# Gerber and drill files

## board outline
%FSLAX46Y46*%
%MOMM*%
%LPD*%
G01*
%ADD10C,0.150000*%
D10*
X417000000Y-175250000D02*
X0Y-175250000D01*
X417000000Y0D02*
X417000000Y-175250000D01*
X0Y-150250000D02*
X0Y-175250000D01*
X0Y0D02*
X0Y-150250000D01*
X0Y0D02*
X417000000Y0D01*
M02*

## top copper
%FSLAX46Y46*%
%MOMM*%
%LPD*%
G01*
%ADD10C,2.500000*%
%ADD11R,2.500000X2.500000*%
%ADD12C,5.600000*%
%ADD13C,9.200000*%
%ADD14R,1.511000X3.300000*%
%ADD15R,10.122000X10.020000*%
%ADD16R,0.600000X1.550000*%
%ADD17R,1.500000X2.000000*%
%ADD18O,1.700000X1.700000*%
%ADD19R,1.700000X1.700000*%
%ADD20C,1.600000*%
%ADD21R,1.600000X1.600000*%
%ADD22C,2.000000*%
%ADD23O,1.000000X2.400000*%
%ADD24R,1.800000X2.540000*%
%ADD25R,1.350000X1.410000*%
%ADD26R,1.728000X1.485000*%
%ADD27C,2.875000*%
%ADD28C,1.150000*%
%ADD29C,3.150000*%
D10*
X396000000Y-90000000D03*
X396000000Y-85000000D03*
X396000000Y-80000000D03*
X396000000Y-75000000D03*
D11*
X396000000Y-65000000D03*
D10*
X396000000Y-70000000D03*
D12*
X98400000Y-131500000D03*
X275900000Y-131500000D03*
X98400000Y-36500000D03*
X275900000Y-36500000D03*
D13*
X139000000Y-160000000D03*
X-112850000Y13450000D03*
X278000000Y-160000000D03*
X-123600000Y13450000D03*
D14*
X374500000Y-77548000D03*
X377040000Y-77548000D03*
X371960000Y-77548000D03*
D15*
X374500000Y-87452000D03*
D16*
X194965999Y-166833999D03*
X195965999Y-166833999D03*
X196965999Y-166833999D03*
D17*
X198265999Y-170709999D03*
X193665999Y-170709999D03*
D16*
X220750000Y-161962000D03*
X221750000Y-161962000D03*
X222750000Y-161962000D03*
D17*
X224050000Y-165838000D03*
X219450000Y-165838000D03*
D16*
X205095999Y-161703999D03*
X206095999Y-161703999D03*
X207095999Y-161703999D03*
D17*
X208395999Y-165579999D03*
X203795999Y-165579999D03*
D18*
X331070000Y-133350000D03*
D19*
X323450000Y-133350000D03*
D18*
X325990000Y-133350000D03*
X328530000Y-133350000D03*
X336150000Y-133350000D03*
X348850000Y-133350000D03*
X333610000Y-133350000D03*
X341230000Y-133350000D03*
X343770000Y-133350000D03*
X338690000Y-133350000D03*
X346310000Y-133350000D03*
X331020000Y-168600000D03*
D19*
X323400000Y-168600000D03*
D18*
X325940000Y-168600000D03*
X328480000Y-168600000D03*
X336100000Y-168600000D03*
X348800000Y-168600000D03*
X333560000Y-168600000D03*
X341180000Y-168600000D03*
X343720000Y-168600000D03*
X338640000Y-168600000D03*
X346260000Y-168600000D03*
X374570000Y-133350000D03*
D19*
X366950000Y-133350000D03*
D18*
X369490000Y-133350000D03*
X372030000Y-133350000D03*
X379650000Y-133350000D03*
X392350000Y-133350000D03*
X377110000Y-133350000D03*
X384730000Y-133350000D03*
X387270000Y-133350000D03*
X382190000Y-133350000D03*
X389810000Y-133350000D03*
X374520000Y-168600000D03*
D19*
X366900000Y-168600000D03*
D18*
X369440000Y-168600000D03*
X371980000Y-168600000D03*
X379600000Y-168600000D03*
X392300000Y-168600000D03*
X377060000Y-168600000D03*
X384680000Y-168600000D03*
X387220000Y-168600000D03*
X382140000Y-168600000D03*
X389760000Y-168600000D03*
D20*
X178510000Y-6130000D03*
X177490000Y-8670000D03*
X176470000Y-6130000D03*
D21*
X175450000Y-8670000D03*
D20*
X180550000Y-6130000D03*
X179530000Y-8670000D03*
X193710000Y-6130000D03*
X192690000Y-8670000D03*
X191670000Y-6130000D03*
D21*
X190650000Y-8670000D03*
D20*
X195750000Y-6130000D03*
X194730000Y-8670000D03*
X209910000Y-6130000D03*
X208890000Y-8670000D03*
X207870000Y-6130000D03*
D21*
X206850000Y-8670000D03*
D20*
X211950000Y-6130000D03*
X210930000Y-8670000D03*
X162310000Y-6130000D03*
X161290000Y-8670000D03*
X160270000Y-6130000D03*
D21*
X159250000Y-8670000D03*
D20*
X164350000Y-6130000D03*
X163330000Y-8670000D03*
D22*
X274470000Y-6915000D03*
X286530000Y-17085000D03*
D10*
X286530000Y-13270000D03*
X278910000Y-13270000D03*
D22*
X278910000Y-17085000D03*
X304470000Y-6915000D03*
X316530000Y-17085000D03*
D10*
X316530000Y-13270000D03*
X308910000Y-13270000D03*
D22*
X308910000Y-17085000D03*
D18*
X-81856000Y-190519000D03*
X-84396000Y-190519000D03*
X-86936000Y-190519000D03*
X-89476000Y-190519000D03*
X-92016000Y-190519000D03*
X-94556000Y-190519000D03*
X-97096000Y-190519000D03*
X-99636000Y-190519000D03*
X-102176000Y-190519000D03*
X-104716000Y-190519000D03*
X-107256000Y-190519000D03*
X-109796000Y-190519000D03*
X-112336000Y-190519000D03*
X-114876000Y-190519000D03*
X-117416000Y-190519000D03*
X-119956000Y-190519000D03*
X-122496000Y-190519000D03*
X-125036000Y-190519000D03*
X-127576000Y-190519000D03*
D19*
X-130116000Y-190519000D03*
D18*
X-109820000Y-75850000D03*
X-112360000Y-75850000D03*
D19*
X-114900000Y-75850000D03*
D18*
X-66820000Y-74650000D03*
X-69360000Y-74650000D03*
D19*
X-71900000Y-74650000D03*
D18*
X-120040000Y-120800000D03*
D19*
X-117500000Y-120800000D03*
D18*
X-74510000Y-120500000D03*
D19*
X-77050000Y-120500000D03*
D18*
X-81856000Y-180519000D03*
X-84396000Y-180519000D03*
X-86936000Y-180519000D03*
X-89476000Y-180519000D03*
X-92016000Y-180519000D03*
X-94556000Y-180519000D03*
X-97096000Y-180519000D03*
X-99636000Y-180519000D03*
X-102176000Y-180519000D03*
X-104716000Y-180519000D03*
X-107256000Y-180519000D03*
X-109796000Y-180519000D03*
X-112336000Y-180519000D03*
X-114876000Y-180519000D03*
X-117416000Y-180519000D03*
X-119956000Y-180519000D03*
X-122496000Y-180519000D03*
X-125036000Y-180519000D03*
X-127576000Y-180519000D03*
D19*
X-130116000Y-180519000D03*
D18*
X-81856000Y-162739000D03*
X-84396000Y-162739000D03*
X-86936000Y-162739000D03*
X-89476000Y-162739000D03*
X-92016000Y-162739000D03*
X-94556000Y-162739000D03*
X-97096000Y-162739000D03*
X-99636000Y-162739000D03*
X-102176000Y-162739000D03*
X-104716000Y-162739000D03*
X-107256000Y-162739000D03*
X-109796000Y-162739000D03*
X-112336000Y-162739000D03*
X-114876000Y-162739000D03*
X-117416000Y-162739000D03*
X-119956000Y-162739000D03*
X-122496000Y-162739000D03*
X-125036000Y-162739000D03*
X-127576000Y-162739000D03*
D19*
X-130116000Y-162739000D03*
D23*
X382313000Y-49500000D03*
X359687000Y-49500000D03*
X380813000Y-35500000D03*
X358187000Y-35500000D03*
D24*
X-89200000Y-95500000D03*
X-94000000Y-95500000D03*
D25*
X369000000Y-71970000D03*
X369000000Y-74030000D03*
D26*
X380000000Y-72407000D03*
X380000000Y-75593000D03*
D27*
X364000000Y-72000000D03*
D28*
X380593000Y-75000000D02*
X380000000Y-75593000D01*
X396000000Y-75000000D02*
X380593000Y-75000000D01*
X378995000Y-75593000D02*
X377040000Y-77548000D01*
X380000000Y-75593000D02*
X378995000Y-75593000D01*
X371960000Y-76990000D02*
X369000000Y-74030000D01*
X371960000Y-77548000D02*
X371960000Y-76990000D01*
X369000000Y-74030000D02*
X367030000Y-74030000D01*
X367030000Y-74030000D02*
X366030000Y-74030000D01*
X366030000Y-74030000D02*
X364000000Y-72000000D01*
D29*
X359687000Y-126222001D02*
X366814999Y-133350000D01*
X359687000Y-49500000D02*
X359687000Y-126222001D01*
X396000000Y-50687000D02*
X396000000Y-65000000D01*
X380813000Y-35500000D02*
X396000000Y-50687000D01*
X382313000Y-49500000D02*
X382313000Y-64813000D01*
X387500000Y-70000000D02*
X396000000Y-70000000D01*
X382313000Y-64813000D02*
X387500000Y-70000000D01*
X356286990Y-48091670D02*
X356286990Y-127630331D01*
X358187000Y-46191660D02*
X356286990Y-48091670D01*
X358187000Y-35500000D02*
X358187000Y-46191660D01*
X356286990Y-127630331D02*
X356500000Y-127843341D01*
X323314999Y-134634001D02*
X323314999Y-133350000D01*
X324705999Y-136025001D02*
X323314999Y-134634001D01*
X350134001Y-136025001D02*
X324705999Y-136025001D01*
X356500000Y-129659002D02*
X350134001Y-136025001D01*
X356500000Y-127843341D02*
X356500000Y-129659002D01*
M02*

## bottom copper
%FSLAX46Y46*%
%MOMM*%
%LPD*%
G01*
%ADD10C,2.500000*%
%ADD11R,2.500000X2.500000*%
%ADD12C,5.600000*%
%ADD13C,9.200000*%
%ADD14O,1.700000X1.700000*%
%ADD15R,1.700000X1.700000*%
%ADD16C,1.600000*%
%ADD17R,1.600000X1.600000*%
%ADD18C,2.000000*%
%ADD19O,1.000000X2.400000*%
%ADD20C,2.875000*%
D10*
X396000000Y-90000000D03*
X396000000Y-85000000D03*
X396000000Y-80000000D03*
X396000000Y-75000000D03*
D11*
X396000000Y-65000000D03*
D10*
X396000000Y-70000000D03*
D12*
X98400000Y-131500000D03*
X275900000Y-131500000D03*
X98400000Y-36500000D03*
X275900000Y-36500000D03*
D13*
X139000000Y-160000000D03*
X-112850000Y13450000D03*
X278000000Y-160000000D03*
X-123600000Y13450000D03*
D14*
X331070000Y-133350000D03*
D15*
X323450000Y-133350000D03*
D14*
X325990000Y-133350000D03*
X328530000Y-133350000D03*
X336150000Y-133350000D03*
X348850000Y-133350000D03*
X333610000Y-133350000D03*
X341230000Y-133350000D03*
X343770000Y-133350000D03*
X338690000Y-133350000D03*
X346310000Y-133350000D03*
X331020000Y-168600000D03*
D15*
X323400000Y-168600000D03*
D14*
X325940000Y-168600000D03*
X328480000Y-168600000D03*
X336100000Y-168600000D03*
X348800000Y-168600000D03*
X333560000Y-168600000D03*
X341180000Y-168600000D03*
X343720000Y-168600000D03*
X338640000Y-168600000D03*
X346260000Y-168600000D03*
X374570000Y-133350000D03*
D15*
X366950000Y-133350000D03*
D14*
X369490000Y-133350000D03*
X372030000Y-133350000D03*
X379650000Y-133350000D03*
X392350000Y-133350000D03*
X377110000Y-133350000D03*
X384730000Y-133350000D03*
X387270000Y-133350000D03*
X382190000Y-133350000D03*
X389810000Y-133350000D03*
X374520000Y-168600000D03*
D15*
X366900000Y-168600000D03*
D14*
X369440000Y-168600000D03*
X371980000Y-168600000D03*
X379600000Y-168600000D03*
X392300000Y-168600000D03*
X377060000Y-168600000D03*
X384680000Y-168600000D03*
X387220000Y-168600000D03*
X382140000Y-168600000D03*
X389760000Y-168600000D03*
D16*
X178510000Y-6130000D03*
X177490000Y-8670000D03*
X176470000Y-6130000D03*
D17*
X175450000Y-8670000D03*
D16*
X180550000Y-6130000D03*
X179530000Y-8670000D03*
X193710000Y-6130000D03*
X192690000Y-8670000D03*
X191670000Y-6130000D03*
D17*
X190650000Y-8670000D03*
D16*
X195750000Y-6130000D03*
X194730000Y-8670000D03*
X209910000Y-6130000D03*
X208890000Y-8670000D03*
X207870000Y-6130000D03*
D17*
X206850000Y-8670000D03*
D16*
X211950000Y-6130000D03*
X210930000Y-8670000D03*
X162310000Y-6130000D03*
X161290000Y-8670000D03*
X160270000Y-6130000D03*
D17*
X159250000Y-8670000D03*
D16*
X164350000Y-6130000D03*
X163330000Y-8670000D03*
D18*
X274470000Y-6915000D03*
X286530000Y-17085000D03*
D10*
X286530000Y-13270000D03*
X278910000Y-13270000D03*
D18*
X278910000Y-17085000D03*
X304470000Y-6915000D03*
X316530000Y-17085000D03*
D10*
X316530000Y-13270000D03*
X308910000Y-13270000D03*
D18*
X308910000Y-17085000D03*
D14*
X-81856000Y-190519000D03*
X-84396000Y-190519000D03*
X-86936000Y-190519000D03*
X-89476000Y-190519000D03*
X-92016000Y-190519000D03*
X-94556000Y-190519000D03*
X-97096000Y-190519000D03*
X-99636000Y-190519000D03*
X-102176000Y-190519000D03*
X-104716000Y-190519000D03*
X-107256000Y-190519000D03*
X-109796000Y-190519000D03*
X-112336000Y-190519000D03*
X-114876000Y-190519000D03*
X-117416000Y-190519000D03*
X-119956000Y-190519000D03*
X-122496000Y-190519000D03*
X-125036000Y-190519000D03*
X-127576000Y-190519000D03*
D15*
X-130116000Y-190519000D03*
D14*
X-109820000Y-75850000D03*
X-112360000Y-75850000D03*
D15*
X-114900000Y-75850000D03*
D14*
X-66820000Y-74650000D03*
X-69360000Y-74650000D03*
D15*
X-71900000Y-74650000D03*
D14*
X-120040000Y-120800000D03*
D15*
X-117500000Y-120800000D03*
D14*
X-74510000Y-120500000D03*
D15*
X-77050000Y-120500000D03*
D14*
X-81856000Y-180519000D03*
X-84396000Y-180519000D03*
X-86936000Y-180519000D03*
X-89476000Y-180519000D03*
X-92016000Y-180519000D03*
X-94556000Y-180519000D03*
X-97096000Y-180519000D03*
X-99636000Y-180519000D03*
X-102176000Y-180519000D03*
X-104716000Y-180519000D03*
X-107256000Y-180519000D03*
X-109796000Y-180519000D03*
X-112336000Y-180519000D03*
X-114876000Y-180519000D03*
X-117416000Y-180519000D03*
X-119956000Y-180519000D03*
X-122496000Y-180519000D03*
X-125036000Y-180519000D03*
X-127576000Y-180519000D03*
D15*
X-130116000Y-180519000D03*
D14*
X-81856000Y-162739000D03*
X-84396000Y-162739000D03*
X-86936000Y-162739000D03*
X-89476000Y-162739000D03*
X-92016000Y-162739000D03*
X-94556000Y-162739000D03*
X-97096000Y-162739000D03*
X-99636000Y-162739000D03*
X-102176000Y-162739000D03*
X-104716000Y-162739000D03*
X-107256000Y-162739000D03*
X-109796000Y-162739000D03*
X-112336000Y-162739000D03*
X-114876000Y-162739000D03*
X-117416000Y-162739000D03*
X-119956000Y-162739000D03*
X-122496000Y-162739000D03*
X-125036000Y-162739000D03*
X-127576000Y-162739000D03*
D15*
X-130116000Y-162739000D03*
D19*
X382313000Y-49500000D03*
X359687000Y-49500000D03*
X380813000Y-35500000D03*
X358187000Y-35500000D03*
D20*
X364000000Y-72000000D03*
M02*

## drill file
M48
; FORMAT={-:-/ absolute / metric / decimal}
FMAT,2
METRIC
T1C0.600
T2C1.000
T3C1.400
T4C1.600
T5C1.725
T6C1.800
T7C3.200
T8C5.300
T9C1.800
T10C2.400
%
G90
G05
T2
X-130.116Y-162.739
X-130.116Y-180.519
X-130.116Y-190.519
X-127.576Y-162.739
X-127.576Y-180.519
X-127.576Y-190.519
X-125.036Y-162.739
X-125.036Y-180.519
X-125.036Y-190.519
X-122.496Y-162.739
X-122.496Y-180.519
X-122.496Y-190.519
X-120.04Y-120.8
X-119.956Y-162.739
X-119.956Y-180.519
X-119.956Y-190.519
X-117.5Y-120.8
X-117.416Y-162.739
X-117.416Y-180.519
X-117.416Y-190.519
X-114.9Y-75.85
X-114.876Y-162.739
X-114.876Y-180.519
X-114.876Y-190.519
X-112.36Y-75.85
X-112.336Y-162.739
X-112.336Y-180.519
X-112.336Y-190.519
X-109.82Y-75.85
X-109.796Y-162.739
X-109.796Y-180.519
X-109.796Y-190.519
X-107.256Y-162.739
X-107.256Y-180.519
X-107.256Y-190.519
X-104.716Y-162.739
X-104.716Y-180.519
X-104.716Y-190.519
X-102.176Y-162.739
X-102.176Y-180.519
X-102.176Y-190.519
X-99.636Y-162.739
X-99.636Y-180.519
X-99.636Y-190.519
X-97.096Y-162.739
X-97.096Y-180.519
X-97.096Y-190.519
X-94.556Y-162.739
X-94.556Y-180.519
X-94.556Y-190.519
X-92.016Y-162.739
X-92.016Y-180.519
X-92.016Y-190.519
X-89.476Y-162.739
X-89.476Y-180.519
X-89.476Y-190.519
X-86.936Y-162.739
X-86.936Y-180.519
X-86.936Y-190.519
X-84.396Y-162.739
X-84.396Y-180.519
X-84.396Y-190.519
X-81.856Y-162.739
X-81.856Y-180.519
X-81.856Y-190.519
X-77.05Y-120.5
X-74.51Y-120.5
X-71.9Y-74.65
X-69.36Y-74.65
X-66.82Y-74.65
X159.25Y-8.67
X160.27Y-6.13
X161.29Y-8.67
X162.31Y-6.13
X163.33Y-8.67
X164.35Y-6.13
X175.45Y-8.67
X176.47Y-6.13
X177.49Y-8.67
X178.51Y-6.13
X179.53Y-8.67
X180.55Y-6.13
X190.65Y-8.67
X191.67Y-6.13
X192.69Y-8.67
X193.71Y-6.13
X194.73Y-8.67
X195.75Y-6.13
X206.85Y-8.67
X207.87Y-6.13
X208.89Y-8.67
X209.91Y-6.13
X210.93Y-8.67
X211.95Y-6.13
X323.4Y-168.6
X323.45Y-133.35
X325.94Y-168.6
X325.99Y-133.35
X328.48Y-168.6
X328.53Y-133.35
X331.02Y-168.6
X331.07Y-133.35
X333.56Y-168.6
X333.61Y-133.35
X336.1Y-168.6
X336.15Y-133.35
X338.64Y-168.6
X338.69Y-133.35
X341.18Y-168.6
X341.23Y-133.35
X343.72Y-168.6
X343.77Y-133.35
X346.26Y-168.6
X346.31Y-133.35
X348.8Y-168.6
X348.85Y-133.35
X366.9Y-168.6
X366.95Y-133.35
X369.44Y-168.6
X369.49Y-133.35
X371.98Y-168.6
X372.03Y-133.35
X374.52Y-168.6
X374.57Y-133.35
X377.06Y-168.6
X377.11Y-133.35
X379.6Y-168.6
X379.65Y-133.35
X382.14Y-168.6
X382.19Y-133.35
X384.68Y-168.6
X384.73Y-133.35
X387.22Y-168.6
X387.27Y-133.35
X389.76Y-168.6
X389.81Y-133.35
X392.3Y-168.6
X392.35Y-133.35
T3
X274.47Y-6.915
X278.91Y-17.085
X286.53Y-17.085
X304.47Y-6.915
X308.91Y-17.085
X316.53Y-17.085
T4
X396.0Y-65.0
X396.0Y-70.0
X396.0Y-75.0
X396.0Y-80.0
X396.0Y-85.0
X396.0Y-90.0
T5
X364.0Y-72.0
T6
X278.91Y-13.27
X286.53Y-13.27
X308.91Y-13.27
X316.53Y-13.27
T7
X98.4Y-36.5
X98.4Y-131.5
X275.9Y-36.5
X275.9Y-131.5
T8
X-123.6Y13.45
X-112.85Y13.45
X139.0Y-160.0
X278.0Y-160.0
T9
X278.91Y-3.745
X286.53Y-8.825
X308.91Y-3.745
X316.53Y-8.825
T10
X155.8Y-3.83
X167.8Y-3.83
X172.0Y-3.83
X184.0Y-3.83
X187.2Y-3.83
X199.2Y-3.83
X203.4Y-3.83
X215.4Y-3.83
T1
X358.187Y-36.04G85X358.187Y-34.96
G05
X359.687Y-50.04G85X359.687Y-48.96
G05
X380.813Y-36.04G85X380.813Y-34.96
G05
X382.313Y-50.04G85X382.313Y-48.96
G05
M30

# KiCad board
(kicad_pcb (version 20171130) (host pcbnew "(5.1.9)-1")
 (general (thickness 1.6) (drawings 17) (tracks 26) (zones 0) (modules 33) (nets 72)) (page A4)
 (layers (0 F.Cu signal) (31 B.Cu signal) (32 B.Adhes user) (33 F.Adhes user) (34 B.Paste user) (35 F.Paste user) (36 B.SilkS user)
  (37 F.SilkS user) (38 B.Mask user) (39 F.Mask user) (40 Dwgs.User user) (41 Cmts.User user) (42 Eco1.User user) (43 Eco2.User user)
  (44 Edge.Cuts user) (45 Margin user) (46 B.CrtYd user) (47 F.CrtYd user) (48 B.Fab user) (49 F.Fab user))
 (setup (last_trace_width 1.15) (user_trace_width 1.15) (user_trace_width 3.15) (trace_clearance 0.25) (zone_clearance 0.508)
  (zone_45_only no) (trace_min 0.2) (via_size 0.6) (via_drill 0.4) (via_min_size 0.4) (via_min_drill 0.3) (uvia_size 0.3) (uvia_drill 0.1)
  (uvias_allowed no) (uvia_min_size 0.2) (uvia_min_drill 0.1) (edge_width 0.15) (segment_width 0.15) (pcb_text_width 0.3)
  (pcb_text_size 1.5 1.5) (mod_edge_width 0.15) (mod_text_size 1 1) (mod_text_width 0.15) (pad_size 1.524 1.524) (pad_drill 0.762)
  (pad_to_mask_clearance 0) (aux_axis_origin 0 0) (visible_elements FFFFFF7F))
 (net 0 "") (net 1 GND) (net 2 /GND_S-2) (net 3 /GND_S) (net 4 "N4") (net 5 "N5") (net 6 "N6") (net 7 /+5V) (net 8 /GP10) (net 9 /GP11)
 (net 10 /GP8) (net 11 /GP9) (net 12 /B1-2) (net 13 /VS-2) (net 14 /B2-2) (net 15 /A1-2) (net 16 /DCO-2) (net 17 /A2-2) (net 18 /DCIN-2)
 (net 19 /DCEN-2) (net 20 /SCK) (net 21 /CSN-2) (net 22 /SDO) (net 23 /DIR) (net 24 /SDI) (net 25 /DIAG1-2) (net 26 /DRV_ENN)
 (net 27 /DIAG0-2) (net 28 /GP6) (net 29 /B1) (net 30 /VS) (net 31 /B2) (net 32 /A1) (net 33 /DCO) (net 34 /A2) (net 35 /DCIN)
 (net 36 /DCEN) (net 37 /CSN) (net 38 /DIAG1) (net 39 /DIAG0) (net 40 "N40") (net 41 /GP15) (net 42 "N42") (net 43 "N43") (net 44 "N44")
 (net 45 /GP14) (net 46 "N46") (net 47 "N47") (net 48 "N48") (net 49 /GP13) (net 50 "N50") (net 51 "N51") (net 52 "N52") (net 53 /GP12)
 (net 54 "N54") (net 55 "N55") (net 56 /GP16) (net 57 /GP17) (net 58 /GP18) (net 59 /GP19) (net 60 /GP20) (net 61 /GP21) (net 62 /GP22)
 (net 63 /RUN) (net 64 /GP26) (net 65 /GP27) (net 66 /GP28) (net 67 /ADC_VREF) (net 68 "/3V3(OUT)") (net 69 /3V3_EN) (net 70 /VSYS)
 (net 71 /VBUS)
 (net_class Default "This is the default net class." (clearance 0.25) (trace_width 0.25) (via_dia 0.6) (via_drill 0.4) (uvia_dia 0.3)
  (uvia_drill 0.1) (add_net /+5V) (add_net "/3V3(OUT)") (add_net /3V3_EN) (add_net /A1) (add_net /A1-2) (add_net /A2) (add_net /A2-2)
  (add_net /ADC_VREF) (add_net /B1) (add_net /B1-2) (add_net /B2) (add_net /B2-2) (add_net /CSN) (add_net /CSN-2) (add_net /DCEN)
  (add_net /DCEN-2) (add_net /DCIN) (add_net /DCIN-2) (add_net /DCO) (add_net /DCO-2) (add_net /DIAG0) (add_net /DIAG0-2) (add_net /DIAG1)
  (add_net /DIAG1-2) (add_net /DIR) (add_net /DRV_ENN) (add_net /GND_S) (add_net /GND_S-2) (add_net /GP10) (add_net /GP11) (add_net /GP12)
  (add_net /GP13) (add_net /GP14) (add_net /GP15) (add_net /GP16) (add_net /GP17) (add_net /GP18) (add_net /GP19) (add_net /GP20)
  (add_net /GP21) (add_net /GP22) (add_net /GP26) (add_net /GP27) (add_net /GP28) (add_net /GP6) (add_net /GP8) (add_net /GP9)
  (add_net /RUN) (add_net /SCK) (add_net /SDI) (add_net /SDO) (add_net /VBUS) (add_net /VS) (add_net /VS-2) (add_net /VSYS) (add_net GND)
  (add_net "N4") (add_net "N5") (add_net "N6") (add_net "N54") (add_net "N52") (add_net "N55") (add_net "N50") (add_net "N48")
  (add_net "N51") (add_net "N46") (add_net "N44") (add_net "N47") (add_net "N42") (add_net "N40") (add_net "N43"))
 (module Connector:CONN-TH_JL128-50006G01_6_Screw (layer F.Cu) (at 396 77.5 270)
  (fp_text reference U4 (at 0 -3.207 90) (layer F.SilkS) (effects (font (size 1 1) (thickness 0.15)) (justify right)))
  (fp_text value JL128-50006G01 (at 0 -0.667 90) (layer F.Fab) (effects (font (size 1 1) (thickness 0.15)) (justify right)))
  (pad 6 thru_hole circle (at 12.5 0 270) (size 2.5 2.5) (drill 1.6) (layers *.Cu *.Mask) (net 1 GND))
  (pad 5 thru_hole circle (at 7.5 0 270) (size 2.5 2.5) (drill 1.6) (layers *.Cu *.Mask) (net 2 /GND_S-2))
  (pad 4 thru_hole circle (at 2.5 0 270) (size 2.5 2.5) (drill 1.6) (layers *.Cu *.Mask) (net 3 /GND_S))
  (pad 3 thru_hole circle (at -2.5 0 270) (size 2.5 2.5) (drill 1.6) (layers *.Cu *.Mask) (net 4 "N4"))
  (pad 1 thru_hole rect (at -12.5 0 270) (size 2.5 2.5) (drill 1.6) (layers *.Cu *.Mask) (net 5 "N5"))
  (pad 2 thru_hole circle (at -7.5 0 270) (size 2.5 2.5) (drill 1.6) (layers *.Cu *.Mask) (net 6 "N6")))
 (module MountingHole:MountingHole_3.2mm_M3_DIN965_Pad (layer F.Cu) (at 98.4 131.5 270)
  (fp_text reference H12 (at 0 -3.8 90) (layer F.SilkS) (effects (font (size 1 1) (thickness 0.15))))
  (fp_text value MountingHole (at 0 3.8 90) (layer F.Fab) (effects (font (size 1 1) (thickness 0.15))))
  (pad 1 thru_hole circle (at 0 0 270) (size 5.6 5.6) (drill 3.2) (layers *.Cu *.Mask)))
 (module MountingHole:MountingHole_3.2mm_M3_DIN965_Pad (layer F.Cu) (at 275.9 131.5 270)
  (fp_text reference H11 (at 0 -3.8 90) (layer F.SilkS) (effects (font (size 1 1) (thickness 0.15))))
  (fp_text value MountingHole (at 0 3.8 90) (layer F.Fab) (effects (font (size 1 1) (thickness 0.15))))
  (pad 1 thru_hole circle (at 0 0 270) (size 5.6 5.6) (drill 3.2) (layers *.Cu *.Mask)))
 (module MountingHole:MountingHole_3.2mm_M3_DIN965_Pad (layer F.Cu) (at 98.4 36.5 270)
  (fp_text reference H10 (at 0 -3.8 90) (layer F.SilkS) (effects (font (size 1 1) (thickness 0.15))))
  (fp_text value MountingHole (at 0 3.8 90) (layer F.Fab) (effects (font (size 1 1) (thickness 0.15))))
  (pad 1 thru_hole circle (at 0 0 270) (size 5.6 5.6) (drill 3.2) (layers *.Cu *.Mask)))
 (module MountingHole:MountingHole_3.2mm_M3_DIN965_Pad (layer F.Cu) (at 275.9 36.5 270)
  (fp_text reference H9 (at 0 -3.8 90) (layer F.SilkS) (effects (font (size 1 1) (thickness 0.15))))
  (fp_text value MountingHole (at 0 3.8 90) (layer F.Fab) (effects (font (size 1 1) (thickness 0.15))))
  (pad 1 thru_hole circle (at 0 0 270) (size 5.6 5.6) (drill 3.2) (layers *.Cu *.Mask)))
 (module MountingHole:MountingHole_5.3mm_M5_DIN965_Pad (layer F.Cu) (at 139 160)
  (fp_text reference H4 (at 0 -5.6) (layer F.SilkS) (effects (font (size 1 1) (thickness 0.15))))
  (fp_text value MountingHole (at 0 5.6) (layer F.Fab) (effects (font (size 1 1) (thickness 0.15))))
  (pad 1 thru_hole circle (at 0 0) (size 9.2 9.2) (drill 5.3) (layers *.Cu *.Mask)))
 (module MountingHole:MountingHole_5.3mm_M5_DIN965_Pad (layer F.Cu) (at -112.85 -13.45)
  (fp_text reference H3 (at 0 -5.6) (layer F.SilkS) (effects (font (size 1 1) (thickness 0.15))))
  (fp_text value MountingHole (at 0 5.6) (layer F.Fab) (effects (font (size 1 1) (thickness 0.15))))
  (pad 1 thru_hole circle (at 0 0) (size 9.2 9.2) (drill 5.3) (layers *.Cu *.Mask)))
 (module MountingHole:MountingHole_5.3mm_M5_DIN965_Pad (layer F.Cu) (at 278 160)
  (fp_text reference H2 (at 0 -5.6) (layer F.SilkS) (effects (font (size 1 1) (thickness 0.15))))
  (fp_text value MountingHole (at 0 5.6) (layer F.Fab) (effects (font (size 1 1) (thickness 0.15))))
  (pad 1 thru_hole circle (at 0 0) (size 9.2 9.2) (drill 5.3) (layers *.Cu *.Mask)))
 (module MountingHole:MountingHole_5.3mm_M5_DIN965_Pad (layer F.Cu) (at -123.6 -13.45)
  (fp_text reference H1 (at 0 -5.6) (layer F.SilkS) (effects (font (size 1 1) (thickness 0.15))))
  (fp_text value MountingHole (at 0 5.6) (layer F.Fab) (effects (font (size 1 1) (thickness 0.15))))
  (pad 1 thru_hole circle (at 0 0) (size 9.2 9.2) (drill 5.3) (layers *.Cu *.Mask)))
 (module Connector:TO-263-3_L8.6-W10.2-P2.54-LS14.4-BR (layer F.Cu) (at 374.5 82.5 90)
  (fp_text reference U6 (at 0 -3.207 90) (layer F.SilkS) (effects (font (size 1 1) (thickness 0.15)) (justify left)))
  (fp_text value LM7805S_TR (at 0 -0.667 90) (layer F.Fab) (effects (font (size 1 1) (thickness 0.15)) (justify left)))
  (pad 2 smd rect (at 4.952 0 90) (size 3.3 1.511) (layers F.Cu F.Paste F.Mask) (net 1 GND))
  (pad 1 smd rect (at 4.952 2.54 90) (size 3.3 1.511) (layers F.Cu F.Paste F.Mask) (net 4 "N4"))
  (pad 3 smd rect (at 4.952 -2.54 90) (size 3.3 1.511) (layers F.Cu F.Paste F.Mask) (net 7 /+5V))
  (pad 4 smd rect (at -4.952 0 90) (size 10.02 10.122) (layers F.Cu F.Paste F.Mask) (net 1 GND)))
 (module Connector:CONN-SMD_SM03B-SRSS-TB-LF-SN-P (layer F.Cu) (at 195.965999 168.771999)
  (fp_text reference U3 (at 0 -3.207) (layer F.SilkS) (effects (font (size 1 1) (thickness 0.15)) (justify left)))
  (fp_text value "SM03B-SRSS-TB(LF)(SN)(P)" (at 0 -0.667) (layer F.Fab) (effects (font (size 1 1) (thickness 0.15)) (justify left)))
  (pad 1 smd rect (at -1 -1.938) (size 0.6 1.55) (layers F.Cu F.Paste F.Mask) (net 7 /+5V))
  (pad 2 smd rect (at 0 -1.938) (size 0.6 1.55) (layers F.Cu F.Paste F.Mask) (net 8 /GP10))
  (pad 3 smd rect (at 1 -1.938) (size 0.6 1.55) (layers F.Cu F.Paste F.Mask) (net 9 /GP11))
  (pad 4 smd rect (at 2.3 1.938) (size 1.5 2) (layers F.Cu F.Paste F.Mask) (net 1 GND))
  (pad 5 smd rect (at -2.3 1.938) (size 1.5 2) (layers F.Cu F.Paste F.Mask) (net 1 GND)))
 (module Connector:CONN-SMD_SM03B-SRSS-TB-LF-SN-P (layer F.Cu) (at 221.75 163.9)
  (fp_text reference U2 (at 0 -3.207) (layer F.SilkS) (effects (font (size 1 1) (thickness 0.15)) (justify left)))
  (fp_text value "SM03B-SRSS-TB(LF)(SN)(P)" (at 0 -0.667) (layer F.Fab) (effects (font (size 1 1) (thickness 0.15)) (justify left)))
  (pad 1 smd rect (at -1 -1.938) (size 0.6 1.55) (layers F.Cu F.Paste F.Mask) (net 7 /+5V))
  (pad 2 smd rect (at 0 -1.938) (size 0.6 1.55) (layers F.Cu F.Paste F.Mask) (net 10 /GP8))
  (pad 3 smd rect (at 1 -1.938) (size 0.6 1.55) (layers F.Cu F.Paste F.Mask) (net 1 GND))
  (pad 4 smd rect (at 2.3 1.938) (size 1.5 2) (layers F.Cu F.Paste F.Mask) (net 1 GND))
  (pad 5 smd rect (at -2.3 1.938) (size 1.5 2) (layers F.Cu F.Paste F.Mask) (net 1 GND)))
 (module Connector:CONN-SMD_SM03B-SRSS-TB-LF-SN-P (layer F.Cu) (at 206.095999 163.641999)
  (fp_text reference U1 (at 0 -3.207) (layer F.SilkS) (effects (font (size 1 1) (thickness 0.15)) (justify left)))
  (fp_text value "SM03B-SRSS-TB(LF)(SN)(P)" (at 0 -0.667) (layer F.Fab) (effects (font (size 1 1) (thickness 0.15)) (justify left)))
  (pad 1 smd rect (at -1 -1.938) (size 0.6 1.55) (layers F.Cu F.Paste F.Mask) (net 7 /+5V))
  (pad 2 smd rect (at 0 -1.938) (size 0.6 1.55) (layers F.Cu F.Paste F.Mask) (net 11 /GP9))
  (pad 3 smd rect (at 1 -1.938) (size 0.6 1.55) (layers F.Cu F.Paste F.Mask) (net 1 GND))
  (pad 4 smd rect (at 2.3 1.938) (size 1.5 2) (layers F.Cu F.Paste F.Mask) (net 1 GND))
  (pad 5 smd rect (at -2.3 1.938) (size 1.5 2) (layers F.Cu F.Paste F.Mask) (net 1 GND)))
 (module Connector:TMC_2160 (layer F.Cu) (at 322 170 90)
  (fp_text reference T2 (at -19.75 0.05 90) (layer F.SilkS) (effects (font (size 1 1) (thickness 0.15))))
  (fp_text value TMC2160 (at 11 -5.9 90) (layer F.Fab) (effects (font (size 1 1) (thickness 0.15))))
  (pad 15 thru_hole oval (at 36.65 9.07 90) (size 1.7 1.7) (drill 1) (layers *.Cu *.Mask) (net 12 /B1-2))
  (pad 12 thru_hole rect (at 36.65 1.45 90) (size 1.7 1.7) (drill 1) (layers *.Cu *.Mask) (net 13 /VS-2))
  (pad 13 thru_hole oval (at 36.65 3.99 90) (size 1.7 1.7) (drill 1) (layers *.Cu *.Mask) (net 2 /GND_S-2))
  (pad 14 thru_hole oval (at 36.65 6.53 90) (size 1.7 1.7) (drill 1) (layers *.Cu *.Mask) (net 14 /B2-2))
  (pad 17 thru_hole oval (at 36.65 14.15 90) (size 1.7 1.7) (drill 1) (layers *.Cu *.Mask) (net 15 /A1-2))
  (pad 22 thru_hole oval (at 36.65 26.85 90) (size 1.7 1.7) (drill 1) (layers *.Cu *.Mask) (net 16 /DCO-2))
  (pad 16 thru_hole oval (at 36.65 11.61 90) (size 1.7 1.7) (drill 1) (layers *.Cu *.Mask) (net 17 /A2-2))
  (pad 19 thru_hole oval (at 36.65 19.23 90) (size 1.7 1.7) (drill 1) (layers *.Cu *.Mask) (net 1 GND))
  (pad 20 thru_hole oval (at 36.65 21.77 90) (size 1.7 1.7) (drill 1) (layers *.Cu *.Mask) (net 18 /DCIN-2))
  (pad 18 thru_hole oval (at 36.65 16.69 90) (size 1.7 1.7) (drill 1) (layers *.Cu *.Mask) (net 1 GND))
  (pad 21 thru_hole oval (at 36.65 24.31 90) (size 1.7 1.7) (drill 1) (layers *.Cu *.Mask) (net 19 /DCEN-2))
  (pad 4 thru_hole oval (at 1.4 9.02 90) (size 1.7 1.7) (drill 1) (layers *.Cu *.Mask) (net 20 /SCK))
  (pad 1 thru_hole rect (at 1.4 1.4 90) (size 1.7 1.7) (drill 1) (layers *.Cu *.Mask) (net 7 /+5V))
  (pad 2 thru_hole oval (at 1.4 3.94 90) (size 1.7 1.7) (drill 1) (layers *.Cu *.Mask) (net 1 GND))
  (pad 3 thru_hole oval (at 1.4 6.48 90) (size 1.7 1.7) (drill 1) (layers *.Cu *.Mask) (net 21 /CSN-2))
  (pad 6 thru_hole oval (at 1.4 14.1 90) (size 1.7 1.7) (drill 1) (layers *.Cu *.Mask) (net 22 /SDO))
  (pad 11 thru_hole oval (at 1.4 26.8 90) (size 1.7 1.7) (drill 1) (layers *.Cu *.Mask) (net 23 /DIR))
  (pad 5 thru_hole oval (at 1.4 11.56 90) (size 1.7 1.7) (drill 1) (layers *.Cu *.Mask) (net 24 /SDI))
  (pad 8 thru_hole oval (at 1.4 19.18 90) (size 1.7 1.7) (drill 1) (layers *.Cu *.Mask) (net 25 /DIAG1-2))
  (pad 9 thru_hole oval (at 1.4 21.72 90) (size 1.7 1.7) (drill 1) (layers *.Cu *.Mask) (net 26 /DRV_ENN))
  (pad 7 thru_hole oval (at 1.4 16.64 90) (size 1.7 1.7) (drill 1) (layers *.Cu *.Mask) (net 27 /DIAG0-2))
  (pad 10 thru_hole oval (at 1.4 24.26 90) (size 1.7 1.7) (drill 1) (layers *.Cu *.Mask) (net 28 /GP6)))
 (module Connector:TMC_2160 (layer F.Cu) (at 365.5 170 90)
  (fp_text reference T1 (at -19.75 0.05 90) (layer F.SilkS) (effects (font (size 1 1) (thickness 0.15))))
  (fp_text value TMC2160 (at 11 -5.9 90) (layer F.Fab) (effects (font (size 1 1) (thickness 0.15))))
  (pad 15 thru_hole oval (at 36.65 9.07 90) (size 1.7 1.7) (drill 1) (layers *.Cu *.Mask) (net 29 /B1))
  (pad 12 thru_hole rect (at 36.65 1.45 90) (size 1.7 1.7) (drill 1) (layers *.Cu *.Mask) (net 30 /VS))
  (pad 13 thru_hole oval (at 36.65 3.99 90) (size 1.7 1.7) (drill 1) (layers *.Cu *.Mask) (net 3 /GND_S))
  (pad 14 thru_hole oval (at 36.65 6.53 90) (size 1.7 1.7) (drill 1) (layers *.Cu *.Mask) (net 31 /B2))
  (pad 17 thru_hole oval (at 36.65 14.15 90) (size 1.7 1.7) (drill 1) (layers *.Cu *.Mask) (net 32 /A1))
  (pad 22 thru_hole oval (at 36.65 26.85 90) (size 1.7 1.7) (drill 1) (layers *.Cu *.Mask) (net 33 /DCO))
  (pad 16 thru_hole oval (at 36.65 11.61 90) (size 1.7 1.7) (drill 1) (layers *.Cu *.Mask) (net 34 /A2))
  (pad 19 thru_hole oval (at 36.65 19.23 90) (size 1.7 1.7) (drill 1) (layers *.Cu *.Mask) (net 1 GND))
  (pad 20 thru_hole oval (at 36.65 21.77 90) (size 1.7 1.7) (drill 1) (layers *.Cu *.Mask) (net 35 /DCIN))
  (pad 18 thru_hole oval (at 36.65 16.69 90) (size 1.7 1.7) (drill 1) (layers *.Cu *.Mask) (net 1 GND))
  (pad 21 thru_hole oval (at 36.65 24.31 90) (size 1.7 1.7) (drill 1) (layers *.Cu *.Mask) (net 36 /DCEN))
  (pad 4 thru_hole oval (at 1.4 9.02 90) (size 1.7 1.7) (drill 1) (layers *.Cu *.Mask) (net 20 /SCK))
  (pad 1 thru_hole rect (at 1.4 1.4 90) (size 1.7 1.7) (drill 1) (layers *.Cu *.Mask) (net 7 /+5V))
  (pad 2 thru_hole oval (at 1.4 3.94 90) (size 1.7 1.7) (drill 1) (layers *.Cu *.Mask) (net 1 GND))
  (pad 3 thru_hole oval (at 1.4 6.48 90) (size 1.7 1.7) (drill 1) (layers *.Cu *.Mask) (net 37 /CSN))
  (pad 6 thru_hole oval (at 1.4 14.1 90) (size 1.7 1.7) (drill 1) (layers *.Cu *.Mask) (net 22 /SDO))
  (pad 11 thru_hole oval (at 1.4 26.8 90) (size 1.7 1.7) (drill 1) (layers *.Cu *.Mask) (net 23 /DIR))
  (pad 5 thru_hole oval (at 1.4 11.56 90) (size 1.7 1.7) (drill 1) (layers *.Cu *.Mask) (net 24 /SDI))
  (pad 8 thru_hole oval (at 1.4 19.18 90) (size 1.7 1.7) (drill 1) (layers *.Cu *.Mask) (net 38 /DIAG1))
  (pad 9 thru_hole oval (at 1.4 21.72 90) (size 1.7 1.7) (drill 1) (layers *.Cu *.Mask) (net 26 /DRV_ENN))
  (pad 7 thru_hole oval (at 1.4 16.64 90) (size 1.7 1.7) (drill 1) (layers *.Cu *.Mask) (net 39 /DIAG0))
  (pad 10 thru_hole oval (at 1.4 24.26 90) (size 1.7 1.7) (drill 1) (layers *.Cu *.Mask) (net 28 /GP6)))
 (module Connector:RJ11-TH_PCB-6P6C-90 (layer F.Cu) (at 178 7.4 180)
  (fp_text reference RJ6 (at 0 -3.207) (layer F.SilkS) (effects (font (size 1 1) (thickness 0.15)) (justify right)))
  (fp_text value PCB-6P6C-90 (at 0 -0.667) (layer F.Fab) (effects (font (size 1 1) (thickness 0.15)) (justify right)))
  (pad "" np_thru_hole circle (at -6 3.57 180) (size 2.4 2.4) (drill 2.4) (layers *.Cu *.Mask))
  (pad "" np_thru_hole circle (at 6 3.57 180) (size 2.4 2.4) (drill 2.4) (layers *.Cu *.Mask))
  (pad 4 thru_hole circle (at -0.51 1.27) (size 1.6 1.6) (drill 1) (layers *.Cu *.Mask) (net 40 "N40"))
  (pad 3 thru_hole circle (at 0.51 -1.27) (size 1.6 1.6) (drill 1) (layers *.Cu *.Mask) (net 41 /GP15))
  (pad 2 thru_hole circle (at 1.53 1.27) (size 1.6 1.6) (drill 1) (layers *.Cu *.Mask) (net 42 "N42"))
  (pad 1 thru_hole rect (at 2.55 -1.27) (size 1.6 1.6) (drill 1) (layers *.Cu *.Mask) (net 7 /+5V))
  (pad 6 thru_hole circle (at -2.55 1.27) (size 1.6 1.6) (drill 1) (layers *.Cu *.Mask) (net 1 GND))
  (pad 5 thru_hole circle (at -1.53 -1.27) (size 1.6 1.6) (drill 1) (layers *.Cu *.Mask) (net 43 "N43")))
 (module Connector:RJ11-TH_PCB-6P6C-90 (layer F.Cu) (at 193.2 7.4 180)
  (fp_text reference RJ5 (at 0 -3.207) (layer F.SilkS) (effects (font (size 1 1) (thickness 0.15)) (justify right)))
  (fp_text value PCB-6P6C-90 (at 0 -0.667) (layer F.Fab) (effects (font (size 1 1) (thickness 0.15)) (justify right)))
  (pad "" np_thru_hole circle (at -6 3.57 180) (size 2.4 2.4) (drill 2.4) (layers *.Cu *.Mask))
  (pad "" np_thru_hole circle (at 6 3.57 180) (size 2.4 2.4) (drill 2.4) (layers *.Cu *.Mask))
  (pad 4 thru_hole circle (at -0.51 1.27) (size 1.6 1.6) (drill 1) (layers *.Cu *.Mask) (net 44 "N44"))
  (pad 3 thru_hole circle (at 0.51 -1.27) (size 1.6 1.6) (drill 1) (layers *.Cu *.Mask) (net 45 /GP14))
  (pad 2 thru_hole circle (at 1.53 1.27) (size 1.6 1.6) (drill 1) (layers *.Cu *.Mask) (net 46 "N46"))
  (pad 1 thru_hole rect (at 2.55 -1.27) (size 1.6 1.6) (drill 1) (layers *.Cu *.Mask) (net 7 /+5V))
  (pad 6 thru_hole circle (at -2.55 1.27) (size 1.6 1.6) (drill 1) (layers *.Cu *.Mask) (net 1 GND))
  (pad 5 thru_hole circle (at -1.53 -1.27) (size 1.6 1.6) (drill 1) (layers *.Cu *.Mask) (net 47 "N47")))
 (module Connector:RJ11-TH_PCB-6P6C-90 (layer F.Cu) (at 209.4 7.4 180)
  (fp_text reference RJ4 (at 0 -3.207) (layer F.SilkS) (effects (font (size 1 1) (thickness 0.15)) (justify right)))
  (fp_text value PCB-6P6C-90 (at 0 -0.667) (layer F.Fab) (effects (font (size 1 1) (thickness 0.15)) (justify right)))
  (pad "" np_thru_hole circle (at -6 3.57 180) (size 2.4 2.4) (drill 2.4) (layers *.Cu *.Mask))
  (pad "" np_thru_hole circle (at 6 3.57 180) (size 2.4 2.4) (drill 2.4) (layers *.Cu *.Mask))
  (pad 4 thru_hole circle (at -0.51 1.27) (size 1.6 1.6) (drill 1) (layers *.Cu *.Mask) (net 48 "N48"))
  (pad 3 thru_hole circle (at 0.51 -1.27) (size 1.6 1.6) (drill 1) (layers *.Cu *.Mask) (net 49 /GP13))
  (pad 2 thru_hole circle (at 1.53 1.27) (size 1.6 1.6) (drill 1) (layers *.Cu *.Mask) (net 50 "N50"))
  (pad 1 thru_hole rect (at 2.55 -1.27) (size 1.6 1.6) (drill 1) (layers *.Cu *.Mask) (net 7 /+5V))
  (pad 6 thru_hole circle (at -2.55 1.27) (size 1.6 1.6) (drill 1) (layers *.Cu *.Mask) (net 1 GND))
  (pad 5 thru_hole circle (at -1.53 -1.27) (size 1.6 1.6) (drill 1) (layers *.Cu *.Mask) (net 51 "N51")))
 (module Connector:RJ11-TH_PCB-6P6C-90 (layer F.Cu) (at 161.8 7.4 180)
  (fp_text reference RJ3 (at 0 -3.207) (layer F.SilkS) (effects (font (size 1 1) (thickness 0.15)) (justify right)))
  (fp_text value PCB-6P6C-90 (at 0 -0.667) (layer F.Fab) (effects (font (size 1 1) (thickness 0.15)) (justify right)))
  (pad "" np_thru_hole circle (at -6 3.57 180) (size 2.4 2.4) (drill 2.4) (layers *.Cu *.Mask))
  (pad "" np_thru_hole circle (at 6 3.57 180) (size 2.4 2.4) (drill 2.4) (layers *.Cu *.Mask))
  (pad 4 thru_hole circle (at -0.51 1.27) (size 1.6 1.6) (drill 1) (layers *.Cu *.Mask) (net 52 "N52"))
  (pad 3 thru_hole circle (at 0.51 -1.27) (size 1.6 1.6) (drill 1) (layers *.Cu *.Mask) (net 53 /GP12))
  (pad 2 thru_hole circle (at 1.53 1.27) (size 1.6 1.6) (drill 1) (layers *.Cu *.Mask) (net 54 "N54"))
  (pad 1 thru_hole rect (at 2.55 -1.27) (size 1.6 1.6) (drill 1) (layers *.Cu *.Mask) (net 7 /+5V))
  (pad 6 thru_hole circle (at -2.55 1.27) (size 1.6 1.6) (drill 1) (layers *.Cu *.Mask) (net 1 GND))
  (pad 5 thru_hole circle (at -1.53 -1.27) (size 1.6 1.6) (drill 1) (layers *.Cu *.Mask) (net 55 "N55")))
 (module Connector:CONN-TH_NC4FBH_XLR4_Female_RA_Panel (layer F.Cu) (at 280.5 12 180)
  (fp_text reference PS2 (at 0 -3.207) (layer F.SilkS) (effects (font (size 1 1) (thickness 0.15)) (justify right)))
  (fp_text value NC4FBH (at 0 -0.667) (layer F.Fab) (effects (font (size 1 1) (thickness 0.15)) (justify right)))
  (pad "" np_thru_hole circle (at -6.03 3.175 180) (size 1.8 1.8) (drill 1.8) (layers *.Cu *.Mask))
  (pad "" np_thru_hole circle (at 1.59 8.255 180) (size 1.8 1.8) (drill 1.8) (layers *.Cu *.Mask))
  (pad 5 thru_hole circle (at 6.03 5.085) (size 2 2) (drill 1.4) (layers *.Cu *.Mask) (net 1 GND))
  (pad 4 thru_hole circle (at -6.03 -5.085) (size 2 2) (drill 1.4) (layers *.Cu *.Mask) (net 14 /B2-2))
  (pad 3 thru_hole circle (at -6.03 -1.27) (size 2.5 2.5) (drill 1.8) (layers *.Cu *.Mask) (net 12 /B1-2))
  (pad 2 thru_hole circle (at 1.59 -1.27) (size 2.5 2.5) (drill 1.8) (layers *.Cu *.Mask) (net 17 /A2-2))
  (pad 1 thru_hole circle (at 1.59 -5.085) (size 2 2) (drill 1.4) (layers *.Cu *.Mask) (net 15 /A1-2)))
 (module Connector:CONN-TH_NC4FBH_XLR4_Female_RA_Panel (layer F.Cu) (at 310.5 12 180)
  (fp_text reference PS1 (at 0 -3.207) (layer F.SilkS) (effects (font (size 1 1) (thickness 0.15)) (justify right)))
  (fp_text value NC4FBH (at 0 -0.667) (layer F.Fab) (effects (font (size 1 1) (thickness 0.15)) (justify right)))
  (pad "" np_thru_hole circle (at -6.03 3.175 180) (size 1.8 1.8) (drill 1.8) (layers *.Cu *.Mask))
  (pad "" np_thru_hole circle (at 1.59 8.255 180) (size 1.8 1.8) (drill 1.8) (layers *.Cu *.Mask))
  (pad 5 thru_hole circle (at 6.03 5.085) (size 2 2) (drill 1.4) (layers *.Cu *.Mask) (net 1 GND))
  (pad 4 thru_hole circle (at -6.03 -5.085) (size 2 2) (drill 1.4) (layers *.Cu *.Mask) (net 31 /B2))
  (pad 3 thru_hole circle (at -6.03 -1.27) (size 2.5 2.5) (drill 1.8) (layers *.Cu *.Mask) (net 29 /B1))
  (pad 2 thru_hole circle (at 1.59 -1.27) (size 2.5 2.5) (drill 1.8) (layers *.Cu *.Mask) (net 34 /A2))
  (pad 1 thru_hole circle (at 1.59 -5.085) (size 2 2) (drill 1.4) (layers *.Cu *.Mask) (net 32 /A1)))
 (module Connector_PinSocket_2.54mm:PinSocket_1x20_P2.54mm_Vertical (layer F.Cu) (at -130.116 190.519 90)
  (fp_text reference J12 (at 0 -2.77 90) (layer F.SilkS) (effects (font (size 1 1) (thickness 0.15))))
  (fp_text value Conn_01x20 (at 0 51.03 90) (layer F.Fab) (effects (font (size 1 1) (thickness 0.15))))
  (pad 20 thru_hole oval (at 0 48.26 90) (size 1.7 1.7) (drill 1) (layers *.Cu *.Mask) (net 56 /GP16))
  (pad 19 thru_hole oval (at 0 45.72 90) (size 1.7 1.7) (drill 1) (layers *.Cu *.Mask) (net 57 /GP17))
  (pad 18 thru_hole oval (at 0 43.18 90) (size 1.7 1.7) (drill 1) (layers *.Cu *.Mask) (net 1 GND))
  (pad 17 thru_hole oval (at 0 40.64 90) (size 1.7 1.7) (drill 1) (layers *.Cu *.Mask) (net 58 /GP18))
  (pad 16 thru_hole oval (at 0 38.1 90) (size 1.7 1.7) (drill 1) (layers *.Cu *.Mask) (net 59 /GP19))
  (pad 15 thru_hole oval (at 0 35.56 90) (size 1.7 1.7) (drill 1) (layers *.Cu *.Mask) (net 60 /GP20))
  (pad 14 thru_hole oval (at 0 33.02 90) (size 1.7 1.7) (drill 1) (layers *.Cu *.Mask) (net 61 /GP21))
  (pad 13 thru_hole oval (at 0 30.48 90) (size 1.7 1.7) (drill 1) (layers *.Cu *.Mask) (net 1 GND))
  (pad 12 thru_hole oval (at 0 27.94 90) (size 1.7 1.7) (drill 1) (layers *.Cu *.Mask) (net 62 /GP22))
  (pad 11 thru_hole oval (at 0 25.4 90) (size 1.7 1.7) (drill 1) (layers *.Cu *.Mask) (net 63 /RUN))
  (pad 10 thru_hole oval (at 0 22.86 90) (size 1.7 1.7) (drill 1) (layers *.Cu *.Mask) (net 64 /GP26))
  (pad 9 thru_hole oval (at 0 20.32 90) (size 1.7 1.7) (drill 1) (layers *.Cu *.Mask) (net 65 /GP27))
  (pad 8 thru_hole oval (at 0 17.78 90) (size 1.7 1.7) (drill 1) (layers *.Cu *.Mask) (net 1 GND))
  (pad 7 thru_hole oval (at 0 15.24 90) (size 1.7 1.7) (drill 1) (layers *.Cu *.Mask) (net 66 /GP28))
  (pad 6 thru_hole oval (at 0 12.7 90) (size 1.7 1.7) (drill 1) (layers *.Cu *.Mask) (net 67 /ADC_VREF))
  (pad 5 thru_hole oval (at 0 10.16 90) (size 1.7 1.7) (drill 1) (layers *.Cu *.Mask) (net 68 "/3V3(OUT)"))
  (pad 4 thru_hole oval (at 0 7.62 90) (size 1.7 1.7) (drill 1) (layers *.Cu *.Mask) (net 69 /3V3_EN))
  (pad 3 thru_hole oval (at 0 5.08 90) (size 1.7 1.7) (drill 1) (layers *.Cu *.Mask) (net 1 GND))
  (pad 2 thru_hole oval (at 0 2.54 90) (size 1.7 1.7) (drill 1) (layers *.Cu *.Mask) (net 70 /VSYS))
  (pad 1 thru_hole rect (at 0 0 90) (size 1.7 1.7) (drill 1) (layers *.Cu *.Mask) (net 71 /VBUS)))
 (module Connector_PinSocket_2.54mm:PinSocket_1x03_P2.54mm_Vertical (layer F.Cu) (at -114.9 75.85 90)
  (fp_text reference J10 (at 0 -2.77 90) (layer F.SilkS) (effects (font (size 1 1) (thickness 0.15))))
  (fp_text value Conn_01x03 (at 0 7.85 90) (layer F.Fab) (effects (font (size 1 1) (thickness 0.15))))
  (pad 3 thru_hole oval (at 0 5.08 90) (size 1.7 1.7) (drill 1) (layers *.Cu *.Mask) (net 16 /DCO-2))
  (pad 2 thru_hole oval (at 0 2.54 90) (size 1.7 1.7) (drill 1) (layers *.Cu *.Mask) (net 19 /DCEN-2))
  (pad 1 thru_hole rect (at 0 0 90) (size 1.7 1.7) (drill 1) (layers *.Cu *.Mask) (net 18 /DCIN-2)))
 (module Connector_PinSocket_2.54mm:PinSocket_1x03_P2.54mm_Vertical (layer F.Cu) (at -71.9 74.65 90)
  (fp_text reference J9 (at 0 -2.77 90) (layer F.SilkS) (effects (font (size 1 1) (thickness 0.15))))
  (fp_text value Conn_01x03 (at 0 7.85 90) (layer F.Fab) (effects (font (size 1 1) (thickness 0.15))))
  (pad 3 thru_hole oval (at 0 5.08 90) (size 1.7 1.7) (drill 1) (layers *.Cu *.Mask) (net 33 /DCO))
  (pad 2 thru_hole oval (at 0 2.54 90) (size 1.7 1.7) (drill 1) (layers *.Cu *.Mask) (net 36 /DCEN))
  (pad 1 thru_hole rect (at 0 0 90) (size 1.7 1.7) (drill 1) (layers *.Cu *.Mask) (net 35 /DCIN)))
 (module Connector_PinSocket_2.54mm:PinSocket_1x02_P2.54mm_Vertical (layer F.Cu) (at -117.5 120.8 270)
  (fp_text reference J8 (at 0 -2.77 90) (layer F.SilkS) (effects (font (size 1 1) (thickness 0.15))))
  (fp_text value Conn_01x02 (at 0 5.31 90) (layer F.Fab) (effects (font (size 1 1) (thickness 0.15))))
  (pad 2 thru_hole oval (at 0 2.54 270) (size 1.7 1.7) (drill 1) (layers *.Cu *.Mask) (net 27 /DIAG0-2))
  (pad 1 thru_hole rect (at 0 0 270) (size 1.7 1.7) (drill 1) (layers *.Cu *.Mask) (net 25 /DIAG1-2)))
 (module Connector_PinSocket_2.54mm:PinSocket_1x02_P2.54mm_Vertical (layer F.Cu) (at -77.05 120.5 90)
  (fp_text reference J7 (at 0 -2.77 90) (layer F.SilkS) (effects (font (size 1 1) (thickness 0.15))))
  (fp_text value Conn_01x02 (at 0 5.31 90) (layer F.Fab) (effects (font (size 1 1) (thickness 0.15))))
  (pad 2 thru_hole oval (at 0 2.54 90) (size 1.7 1.7) (drill 1) (layers *.Cu *.Mask) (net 38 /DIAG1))
  (pad 1 thru_hole rect (at 0 0 90) (size 1.7 1.7) (drill 1) (layers *.Cu *.Mask) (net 39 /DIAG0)))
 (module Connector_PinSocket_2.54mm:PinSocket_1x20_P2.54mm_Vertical (layer F.Cu) (at -130.116 180.519 90)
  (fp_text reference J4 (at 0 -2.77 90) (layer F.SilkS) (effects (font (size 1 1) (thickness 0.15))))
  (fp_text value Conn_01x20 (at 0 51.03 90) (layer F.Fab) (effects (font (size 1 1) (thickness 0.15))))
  (pad 20 thru_hole oval (at 0 48.26 90) (size 1.7 1.7) (drill 1) (layers *.Cu *.Mask) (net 56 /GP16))
  (pad 19 thru_hole oval (at 0 45.72 90) (size 1.7 1.7) (drill 1) (layers *.Cu *.Mask) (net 57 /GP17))
  (pad 18 thru_hole oval (at 0 43.18 90) (size 1.7 1.7) (drill 1) (layers *.Cu *.Mask) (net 1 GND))
  (pad 17 thru_hole oval (at 0 40.64 90) (size 1.7 1.7) (drill 1) (layers *.Cu *.Mask) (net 58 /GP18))
  (pad 16 thru_hole oval (at 0 38.1 90) (size 1.7 1.7) (drill 1) (layers *.Cu *.Mask) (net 59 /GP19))
  (pad 15 thru_hole oval (at 0 35.56 90) (size 1.7 1.7) (drill 1) (layers *.Cu *.Mask) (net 60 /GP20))
  (pad 14 thru_hole oval (at 0 33.02 90) (size 1.7 1.7) (drill 1) (layers *.Cu *.Mask) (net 61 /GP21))
  (pad 13 thru_hole oval (at 0 30.48 90) (size 1.7 1.7) (drill 1) (layers *.Cu *.Mask) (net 1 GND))
  (pad 12 thru_hole oval (at 0 27.94 90) (size 1.7 1.7) (drill 1) (layers *.Cu *.Mask) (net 62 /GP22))
  (pad 11 thru_hole oval (at 0 25.4 90) (size 1.7 1.7) (drill 1) (layers *.Cu *.Mask) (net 63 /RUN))
  (pad 10 thru_hole oval (at 0 22.86 90) (size 1.7 1.7) (drill 1) (layers *.Cu *.Mask) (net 64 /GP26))
  (pad 9 thru_hole oval (at 0 20.32 90) (size 1.7 1.7) (drill 1) (layers *.Cu *.Mask) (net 65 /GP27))
  (pad 8 thru_hole oval (at 0 17.78 90) (size 1.7 1.7) (drill 1) (layers *.Cu *.Mask) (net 1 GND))
  (pad 7 thru_hole oval (at 0 15.24 90) (size 1.7 1.7) (drill 1) (layers *.Cu *.Mask) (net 66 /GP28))
  (pad 6 thru_hole oval (at 0 12.7 90) (size 1.7 1.7) (drill 1) (layers *.Cu *.Mask) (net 67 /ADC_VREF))
  (pad 5 thru_hole oval (at 0 10.16 90) (size 1.7 1.7) (drill 1) (layers *.Cu *.Mask) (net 68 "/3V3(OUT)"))
  (pad 4 thru_hole oval (at 0 7.62 90) (size 1.7 1.7) (drill 1) (layers *.Cu *.Mask) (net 69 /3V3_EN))
  (pad 3 thru_hole oval (at 0 5.08 90) (size 1.7 1.7) (drill 1) (layers *.Cu *.Mask) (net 1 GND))
  (pad 2 thru_hole oval (at 0 2.54 90) (size 1.7 1.7) (drill 1) (layers *.Cu *.Mask) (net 70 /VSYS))
  (pad 1 thru_hole rect (at 0 0 90) (size 1.7 1.7) (drill 1) (layers *.Cu *.Mask) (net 71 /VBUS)))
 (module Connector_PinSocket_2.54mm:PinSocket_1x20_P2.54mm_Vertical (layer F.Cu) (at -130.116 162.739 90)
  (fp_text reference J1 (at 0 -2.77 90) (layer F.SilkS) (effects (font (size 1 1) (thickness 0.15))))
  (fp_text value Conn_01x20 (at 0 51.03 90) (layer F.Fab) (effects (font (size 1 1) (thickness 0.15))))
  (pad 20 thru_hole oval (at 0 48.26 90) (size 1.7 1.7) (drill 1) (layers *.Cu *.Mask) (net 41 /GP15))
  (pad 19 thru_hole oval (at 0 45.72 90) (size 1.7 1.7) (drill 1) (layers *.Cu *.Mask) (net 45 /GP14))
  (pad 18 thru_hole oval (at 0 43.18 90) (size 1.7 1.7) (drill 1) (layers *.Cu *.Mask) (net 1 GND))
  (pad 17 thru_hole oval (at 0 40.64 90) (size 1.7 1.7) (drill 1) (layers *.Cu *.Mask) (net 49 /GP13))
  (pad 16 thru_hole oval (at 0 38.1 90) (size 1.7 1.7) (drill 1) (layers *.Cu *.Mask) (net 53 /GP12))
  (pad 15 thru_hole oval (at 0 35.56 90) (size 1.7 1.7) (drill 1) (layers *.Cu *.Mask) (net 9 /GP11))
  (pad 14 thru_hole oval (at 0 33.02 90) (size 1.7 1.7) (drill 1) (layers *.Cu *.Mask) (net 8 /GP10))
  (pad 13 thru_hole oval (at 0 30.48 90) (size 1.7 1.7) (drill 1) (layers *.Cu *.Mask) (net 1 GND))
  (pad 12 thru_hole oval (at 0 27.94 90) (size 1.7 1.7) (drill 1) (layers *.Cu *.Mask) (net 11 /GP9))
  (pad 11 thru_hole oval (at 0 25.4 90) (size 1.7 1.7) (drill 1) (layers *.Cu *.Mask) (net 10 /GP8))
  (pad 10 thru_hole oval (at 0 22.86 90) (size 1.7 1.7) (drill 1) (layers *.Cu *.Mask) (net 23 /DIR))
  (pad 9 thru_hole oval (at 0 20.32 90) (size 1.7 1.7) (drill 1) (layers *.Cu *.Mask) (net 28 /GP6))
  (pad 8 thru_hole oval (at 0 17.78 90) (size 1.7 1.7) (drill 1) (layers *.Cu *.Mask) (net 1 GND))
  (pad 7 thru_hole oval (at 0 15.24 90) (size 1.7 1.7) (drill 1) (layers *.Cu *.Mask) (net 21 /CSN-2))
  (pad 6 thru_hole oval (at 0 12.7 90) (size 1.7 1.7) (drill 1) (layers *.Cu *.Mask) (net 26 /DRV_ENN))
  (pad 5 thru_hole oval (at 0 10.16 90) (size 1.7 1.7) (drill 1) (layers *.Cu *.Mask) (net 24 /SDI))
  (pad 4 thru_hole oval (at 0 7.62 90) (size 1.7 1.7) (drill 1) (layers *.Cu *.Mask) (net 20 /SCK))
  (pad 3 thru_hole oval (at 0 5.08 90) (size 1.7 1.7) (drill 1) (layers *.Cu *.Mask) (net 1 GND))
  (pad 2 thru_hole oval (at 0 2.54 90) (size 1.7 1.7) (drill 1) (layers *.Cu *.Mask) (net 37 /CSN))
  (pad 1 thru_hole rect (at 0 0 90) (size 1.7 1.7) (drill 1) (layers *.Cu *.Mask) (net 22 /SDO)))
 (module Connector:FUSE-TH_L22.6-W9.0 (layer F.Cu) (at 371 49.5 180)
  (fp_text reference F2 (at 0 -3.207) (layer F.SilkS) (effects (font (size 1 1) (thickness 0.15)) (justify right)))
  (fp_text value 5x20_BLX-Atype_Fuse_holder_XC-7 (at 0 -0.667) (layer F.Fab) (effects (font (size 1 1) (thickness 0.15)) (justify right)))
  (pad 1 thru_hole oval (at -11.313 0 180) (size 1 2.4) (drill oval 0.6 1.68) (layers *.Cu *.Mask) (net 6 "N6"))
  (pad 2 thru_hole oval (at 11.313 0 180) (size 1 2.4) (drill oval 0.6 1.68) (layers *.Cu *.Mask) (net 30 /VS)))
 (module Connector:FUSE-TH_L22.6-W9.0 (layer F.Cu) (at 369.5 35.5 180)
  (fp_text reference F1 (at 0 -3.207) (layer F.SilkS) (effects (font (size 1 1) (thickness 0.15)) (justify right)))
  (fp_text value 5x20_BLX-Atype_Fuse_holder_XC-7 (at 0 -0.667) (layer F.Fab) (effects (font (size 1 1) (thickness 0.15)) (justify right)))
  (pad 1 thru_hole oval (at -11.313 0 180) (size 1 2.4) (drill oval 0.6 1.68) (layers *.Cu *.Mask) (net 5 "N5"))
  (pad 2 thru_hole oval (at 11.313 0 180) (size 1 2.4) (drill oval 0.6 1.68) (layers *.Cu *.Mask) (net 13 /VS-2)))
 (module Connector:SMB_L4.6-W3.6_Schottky (layer F.Cu) (at -91.6 95.5)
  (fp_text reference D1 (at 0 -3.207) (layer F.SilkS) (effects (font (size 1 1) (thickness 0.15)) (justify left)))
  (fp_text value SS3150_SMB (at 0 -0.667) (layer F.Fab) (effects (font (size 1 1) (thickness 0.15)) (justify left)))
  (pad 1 smd rect (at 2.4 0) (size 1.8 2.54) (layers F.Cu F.Paste F.Mask) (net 7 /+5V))
  (pad 2 smd rect (at -2.4 0) (size 1.8 2.54) (layers F.Cu F.Paste F.Mask) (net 70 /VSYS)))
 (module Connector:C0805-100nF (layer F.Cu) (at 369 73 90)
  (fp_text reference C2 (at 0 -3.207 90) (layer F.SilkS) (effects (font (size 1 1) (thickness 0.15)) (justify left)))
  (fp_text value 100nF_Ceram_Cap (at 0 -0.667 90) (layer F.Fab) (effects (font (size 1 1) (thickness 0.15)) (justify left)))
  (pad 2 smd rect (at 1.03 0 90) (size 1.41 1.35) (layers F.Cu F.Paste F.Mask) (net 1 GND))
  (pad 1 smd rect (at -1.03 0 90) (size 1.41 1.35) (layers F.Cu F.Paste F.Mask) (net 7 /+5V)))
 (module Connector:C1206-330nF (layer F.Cu) (at 380 74 90)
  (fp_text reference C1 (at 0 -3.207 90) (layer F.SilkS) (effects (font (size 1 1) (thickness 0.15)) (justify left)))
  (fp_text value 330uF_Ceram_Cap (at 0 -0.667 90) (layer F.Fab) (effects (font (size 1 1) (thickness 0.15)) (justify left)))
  (pad 2 smd rect (at 1.593 0 90) (size 1.485 1.728) (layers F.Cu F.Paste F.Mask) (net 1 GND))
  (pad 1 smd rect (at -1.593 0 90) (size 1.485 1.728) (layers F.Cu F.Paste F.Mask) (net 4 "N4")))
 (gr_line (start 417 175.25) (end 0 175.25) (layer Edge.Cuts) (width 0.15))
 (gr_line (start 417 0) (end 417 175.25) (layer Edge.Cuts) (width 0.15))
 (gr_line (start 0 150.25) (end 0 175.25) (layer Edge.Cuts) (width 0.15))
 (gr_line (start 0 0) (end 0 150.25) (layer Edge.Cuts) (width 0.15))
 (gr_line (start 0 0) (end 417 0) (layer Edge.Cuts) (width 0.15))
 (via (at 364 72) (size 2.875) (drill 1.725) (layers F.Cu B.Cu) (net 7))
 (segment (start 380.593 75) (end 380 75.593) (width 1.15) (layer F.Cu) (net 4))
 (segment (start 396 75) (end 380.593 75) (width 1.15) (layer F.Cu) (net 4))
 (segment (start 378.995 75.593) (end 377.04 77.548) (width 1.15) (layer F.Cu) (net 4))
 (segment (start 380 75.593) (end 378.995 75.593) (width 1.15) (layer F.Cu) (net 4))
 (segment (start 371.96 76.99) (end 369 74.03) (width 1.15) (layer F.Cu) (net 7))
 (segment (start 371.96 77.548) (end 371.96 76.99) (width 1.15) (layer F.Cu) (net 7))
 (segment (start 369 74.03) (end 367.03 74.03) (width 1.15) (layer F.Cu) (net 7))
 (segment (start 367.03 74.03) (end 366.03 74.03) (width 1.15) (layer F.Cu) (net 7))
 (segment (start 366.03 74.03) (end 364 72) (width 1.15) (layer F.Cu) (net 7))
 (segment (start 359.687 126.222001) (end 366.814999 133.35) (width 3.15) (layer F.Cu) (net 30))
 (segment (start 359.687 49.5) (end 359.687 126.222001) (width 3.15) (layer F.Cu) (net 30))
 (segment (start 396 50.687) (end 396 65) (width 3.15) (layer F.Cu) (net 5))
 (segment (start 380.813 35.5) (end 396 50.687) (width 3.15) (layer F.Cu) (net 5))
 (segment (start 382.313 49.5) (end 382.313 64.813) (width 3.15) (layer F.Cu) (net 6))
 (segment (start 387.5 70) (end 396 70) (width 3.15) (layer F.Cu) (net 6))
 (segment (start 382.313 64.813) (end 387.5 70) (width 3.15) (layer F.Cu) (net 6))
 (segment (start 356.28699 48.09167) (end 356.28699 127.630331) (width 3.15) (layer F.Cu) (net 13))
 (segment (start 358.187 46.19166) (end 356.28699 48.09167) (width 3.15) (layer F.Cu) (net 13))
 (segment (start 358.187 35.5) (end 358.187 46.19166) (width 3.15) (layer F.Cu) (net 13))
 (segment (start 356.28699 127.630331) (end 356.5 127.843341) (width 3.15) (layer F.Cu) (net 13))
 (segment (start 323.314999 134.634001) (end 323.314999 133.35) (width 3.15) (layer F.Cu) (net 13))
 (segment (start 324.705999 136.025001) (end 323.314999 134.634001) (width 3.15) (layer F.Cu) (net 13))
 (segment (start 350.134001 136.025001) (end 324.705999 136.025001) (width 3.15) (layer F.Cu) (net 13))
 (segment (start 356.5 129.659002) (end 350.134001 136.025001) (width 3.15) (layer F.Cu) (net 13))
 (segment (start 356.5 127.843341) (end 356.5 129.659002) (width 3.15) (layer F.Cu) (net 13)))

